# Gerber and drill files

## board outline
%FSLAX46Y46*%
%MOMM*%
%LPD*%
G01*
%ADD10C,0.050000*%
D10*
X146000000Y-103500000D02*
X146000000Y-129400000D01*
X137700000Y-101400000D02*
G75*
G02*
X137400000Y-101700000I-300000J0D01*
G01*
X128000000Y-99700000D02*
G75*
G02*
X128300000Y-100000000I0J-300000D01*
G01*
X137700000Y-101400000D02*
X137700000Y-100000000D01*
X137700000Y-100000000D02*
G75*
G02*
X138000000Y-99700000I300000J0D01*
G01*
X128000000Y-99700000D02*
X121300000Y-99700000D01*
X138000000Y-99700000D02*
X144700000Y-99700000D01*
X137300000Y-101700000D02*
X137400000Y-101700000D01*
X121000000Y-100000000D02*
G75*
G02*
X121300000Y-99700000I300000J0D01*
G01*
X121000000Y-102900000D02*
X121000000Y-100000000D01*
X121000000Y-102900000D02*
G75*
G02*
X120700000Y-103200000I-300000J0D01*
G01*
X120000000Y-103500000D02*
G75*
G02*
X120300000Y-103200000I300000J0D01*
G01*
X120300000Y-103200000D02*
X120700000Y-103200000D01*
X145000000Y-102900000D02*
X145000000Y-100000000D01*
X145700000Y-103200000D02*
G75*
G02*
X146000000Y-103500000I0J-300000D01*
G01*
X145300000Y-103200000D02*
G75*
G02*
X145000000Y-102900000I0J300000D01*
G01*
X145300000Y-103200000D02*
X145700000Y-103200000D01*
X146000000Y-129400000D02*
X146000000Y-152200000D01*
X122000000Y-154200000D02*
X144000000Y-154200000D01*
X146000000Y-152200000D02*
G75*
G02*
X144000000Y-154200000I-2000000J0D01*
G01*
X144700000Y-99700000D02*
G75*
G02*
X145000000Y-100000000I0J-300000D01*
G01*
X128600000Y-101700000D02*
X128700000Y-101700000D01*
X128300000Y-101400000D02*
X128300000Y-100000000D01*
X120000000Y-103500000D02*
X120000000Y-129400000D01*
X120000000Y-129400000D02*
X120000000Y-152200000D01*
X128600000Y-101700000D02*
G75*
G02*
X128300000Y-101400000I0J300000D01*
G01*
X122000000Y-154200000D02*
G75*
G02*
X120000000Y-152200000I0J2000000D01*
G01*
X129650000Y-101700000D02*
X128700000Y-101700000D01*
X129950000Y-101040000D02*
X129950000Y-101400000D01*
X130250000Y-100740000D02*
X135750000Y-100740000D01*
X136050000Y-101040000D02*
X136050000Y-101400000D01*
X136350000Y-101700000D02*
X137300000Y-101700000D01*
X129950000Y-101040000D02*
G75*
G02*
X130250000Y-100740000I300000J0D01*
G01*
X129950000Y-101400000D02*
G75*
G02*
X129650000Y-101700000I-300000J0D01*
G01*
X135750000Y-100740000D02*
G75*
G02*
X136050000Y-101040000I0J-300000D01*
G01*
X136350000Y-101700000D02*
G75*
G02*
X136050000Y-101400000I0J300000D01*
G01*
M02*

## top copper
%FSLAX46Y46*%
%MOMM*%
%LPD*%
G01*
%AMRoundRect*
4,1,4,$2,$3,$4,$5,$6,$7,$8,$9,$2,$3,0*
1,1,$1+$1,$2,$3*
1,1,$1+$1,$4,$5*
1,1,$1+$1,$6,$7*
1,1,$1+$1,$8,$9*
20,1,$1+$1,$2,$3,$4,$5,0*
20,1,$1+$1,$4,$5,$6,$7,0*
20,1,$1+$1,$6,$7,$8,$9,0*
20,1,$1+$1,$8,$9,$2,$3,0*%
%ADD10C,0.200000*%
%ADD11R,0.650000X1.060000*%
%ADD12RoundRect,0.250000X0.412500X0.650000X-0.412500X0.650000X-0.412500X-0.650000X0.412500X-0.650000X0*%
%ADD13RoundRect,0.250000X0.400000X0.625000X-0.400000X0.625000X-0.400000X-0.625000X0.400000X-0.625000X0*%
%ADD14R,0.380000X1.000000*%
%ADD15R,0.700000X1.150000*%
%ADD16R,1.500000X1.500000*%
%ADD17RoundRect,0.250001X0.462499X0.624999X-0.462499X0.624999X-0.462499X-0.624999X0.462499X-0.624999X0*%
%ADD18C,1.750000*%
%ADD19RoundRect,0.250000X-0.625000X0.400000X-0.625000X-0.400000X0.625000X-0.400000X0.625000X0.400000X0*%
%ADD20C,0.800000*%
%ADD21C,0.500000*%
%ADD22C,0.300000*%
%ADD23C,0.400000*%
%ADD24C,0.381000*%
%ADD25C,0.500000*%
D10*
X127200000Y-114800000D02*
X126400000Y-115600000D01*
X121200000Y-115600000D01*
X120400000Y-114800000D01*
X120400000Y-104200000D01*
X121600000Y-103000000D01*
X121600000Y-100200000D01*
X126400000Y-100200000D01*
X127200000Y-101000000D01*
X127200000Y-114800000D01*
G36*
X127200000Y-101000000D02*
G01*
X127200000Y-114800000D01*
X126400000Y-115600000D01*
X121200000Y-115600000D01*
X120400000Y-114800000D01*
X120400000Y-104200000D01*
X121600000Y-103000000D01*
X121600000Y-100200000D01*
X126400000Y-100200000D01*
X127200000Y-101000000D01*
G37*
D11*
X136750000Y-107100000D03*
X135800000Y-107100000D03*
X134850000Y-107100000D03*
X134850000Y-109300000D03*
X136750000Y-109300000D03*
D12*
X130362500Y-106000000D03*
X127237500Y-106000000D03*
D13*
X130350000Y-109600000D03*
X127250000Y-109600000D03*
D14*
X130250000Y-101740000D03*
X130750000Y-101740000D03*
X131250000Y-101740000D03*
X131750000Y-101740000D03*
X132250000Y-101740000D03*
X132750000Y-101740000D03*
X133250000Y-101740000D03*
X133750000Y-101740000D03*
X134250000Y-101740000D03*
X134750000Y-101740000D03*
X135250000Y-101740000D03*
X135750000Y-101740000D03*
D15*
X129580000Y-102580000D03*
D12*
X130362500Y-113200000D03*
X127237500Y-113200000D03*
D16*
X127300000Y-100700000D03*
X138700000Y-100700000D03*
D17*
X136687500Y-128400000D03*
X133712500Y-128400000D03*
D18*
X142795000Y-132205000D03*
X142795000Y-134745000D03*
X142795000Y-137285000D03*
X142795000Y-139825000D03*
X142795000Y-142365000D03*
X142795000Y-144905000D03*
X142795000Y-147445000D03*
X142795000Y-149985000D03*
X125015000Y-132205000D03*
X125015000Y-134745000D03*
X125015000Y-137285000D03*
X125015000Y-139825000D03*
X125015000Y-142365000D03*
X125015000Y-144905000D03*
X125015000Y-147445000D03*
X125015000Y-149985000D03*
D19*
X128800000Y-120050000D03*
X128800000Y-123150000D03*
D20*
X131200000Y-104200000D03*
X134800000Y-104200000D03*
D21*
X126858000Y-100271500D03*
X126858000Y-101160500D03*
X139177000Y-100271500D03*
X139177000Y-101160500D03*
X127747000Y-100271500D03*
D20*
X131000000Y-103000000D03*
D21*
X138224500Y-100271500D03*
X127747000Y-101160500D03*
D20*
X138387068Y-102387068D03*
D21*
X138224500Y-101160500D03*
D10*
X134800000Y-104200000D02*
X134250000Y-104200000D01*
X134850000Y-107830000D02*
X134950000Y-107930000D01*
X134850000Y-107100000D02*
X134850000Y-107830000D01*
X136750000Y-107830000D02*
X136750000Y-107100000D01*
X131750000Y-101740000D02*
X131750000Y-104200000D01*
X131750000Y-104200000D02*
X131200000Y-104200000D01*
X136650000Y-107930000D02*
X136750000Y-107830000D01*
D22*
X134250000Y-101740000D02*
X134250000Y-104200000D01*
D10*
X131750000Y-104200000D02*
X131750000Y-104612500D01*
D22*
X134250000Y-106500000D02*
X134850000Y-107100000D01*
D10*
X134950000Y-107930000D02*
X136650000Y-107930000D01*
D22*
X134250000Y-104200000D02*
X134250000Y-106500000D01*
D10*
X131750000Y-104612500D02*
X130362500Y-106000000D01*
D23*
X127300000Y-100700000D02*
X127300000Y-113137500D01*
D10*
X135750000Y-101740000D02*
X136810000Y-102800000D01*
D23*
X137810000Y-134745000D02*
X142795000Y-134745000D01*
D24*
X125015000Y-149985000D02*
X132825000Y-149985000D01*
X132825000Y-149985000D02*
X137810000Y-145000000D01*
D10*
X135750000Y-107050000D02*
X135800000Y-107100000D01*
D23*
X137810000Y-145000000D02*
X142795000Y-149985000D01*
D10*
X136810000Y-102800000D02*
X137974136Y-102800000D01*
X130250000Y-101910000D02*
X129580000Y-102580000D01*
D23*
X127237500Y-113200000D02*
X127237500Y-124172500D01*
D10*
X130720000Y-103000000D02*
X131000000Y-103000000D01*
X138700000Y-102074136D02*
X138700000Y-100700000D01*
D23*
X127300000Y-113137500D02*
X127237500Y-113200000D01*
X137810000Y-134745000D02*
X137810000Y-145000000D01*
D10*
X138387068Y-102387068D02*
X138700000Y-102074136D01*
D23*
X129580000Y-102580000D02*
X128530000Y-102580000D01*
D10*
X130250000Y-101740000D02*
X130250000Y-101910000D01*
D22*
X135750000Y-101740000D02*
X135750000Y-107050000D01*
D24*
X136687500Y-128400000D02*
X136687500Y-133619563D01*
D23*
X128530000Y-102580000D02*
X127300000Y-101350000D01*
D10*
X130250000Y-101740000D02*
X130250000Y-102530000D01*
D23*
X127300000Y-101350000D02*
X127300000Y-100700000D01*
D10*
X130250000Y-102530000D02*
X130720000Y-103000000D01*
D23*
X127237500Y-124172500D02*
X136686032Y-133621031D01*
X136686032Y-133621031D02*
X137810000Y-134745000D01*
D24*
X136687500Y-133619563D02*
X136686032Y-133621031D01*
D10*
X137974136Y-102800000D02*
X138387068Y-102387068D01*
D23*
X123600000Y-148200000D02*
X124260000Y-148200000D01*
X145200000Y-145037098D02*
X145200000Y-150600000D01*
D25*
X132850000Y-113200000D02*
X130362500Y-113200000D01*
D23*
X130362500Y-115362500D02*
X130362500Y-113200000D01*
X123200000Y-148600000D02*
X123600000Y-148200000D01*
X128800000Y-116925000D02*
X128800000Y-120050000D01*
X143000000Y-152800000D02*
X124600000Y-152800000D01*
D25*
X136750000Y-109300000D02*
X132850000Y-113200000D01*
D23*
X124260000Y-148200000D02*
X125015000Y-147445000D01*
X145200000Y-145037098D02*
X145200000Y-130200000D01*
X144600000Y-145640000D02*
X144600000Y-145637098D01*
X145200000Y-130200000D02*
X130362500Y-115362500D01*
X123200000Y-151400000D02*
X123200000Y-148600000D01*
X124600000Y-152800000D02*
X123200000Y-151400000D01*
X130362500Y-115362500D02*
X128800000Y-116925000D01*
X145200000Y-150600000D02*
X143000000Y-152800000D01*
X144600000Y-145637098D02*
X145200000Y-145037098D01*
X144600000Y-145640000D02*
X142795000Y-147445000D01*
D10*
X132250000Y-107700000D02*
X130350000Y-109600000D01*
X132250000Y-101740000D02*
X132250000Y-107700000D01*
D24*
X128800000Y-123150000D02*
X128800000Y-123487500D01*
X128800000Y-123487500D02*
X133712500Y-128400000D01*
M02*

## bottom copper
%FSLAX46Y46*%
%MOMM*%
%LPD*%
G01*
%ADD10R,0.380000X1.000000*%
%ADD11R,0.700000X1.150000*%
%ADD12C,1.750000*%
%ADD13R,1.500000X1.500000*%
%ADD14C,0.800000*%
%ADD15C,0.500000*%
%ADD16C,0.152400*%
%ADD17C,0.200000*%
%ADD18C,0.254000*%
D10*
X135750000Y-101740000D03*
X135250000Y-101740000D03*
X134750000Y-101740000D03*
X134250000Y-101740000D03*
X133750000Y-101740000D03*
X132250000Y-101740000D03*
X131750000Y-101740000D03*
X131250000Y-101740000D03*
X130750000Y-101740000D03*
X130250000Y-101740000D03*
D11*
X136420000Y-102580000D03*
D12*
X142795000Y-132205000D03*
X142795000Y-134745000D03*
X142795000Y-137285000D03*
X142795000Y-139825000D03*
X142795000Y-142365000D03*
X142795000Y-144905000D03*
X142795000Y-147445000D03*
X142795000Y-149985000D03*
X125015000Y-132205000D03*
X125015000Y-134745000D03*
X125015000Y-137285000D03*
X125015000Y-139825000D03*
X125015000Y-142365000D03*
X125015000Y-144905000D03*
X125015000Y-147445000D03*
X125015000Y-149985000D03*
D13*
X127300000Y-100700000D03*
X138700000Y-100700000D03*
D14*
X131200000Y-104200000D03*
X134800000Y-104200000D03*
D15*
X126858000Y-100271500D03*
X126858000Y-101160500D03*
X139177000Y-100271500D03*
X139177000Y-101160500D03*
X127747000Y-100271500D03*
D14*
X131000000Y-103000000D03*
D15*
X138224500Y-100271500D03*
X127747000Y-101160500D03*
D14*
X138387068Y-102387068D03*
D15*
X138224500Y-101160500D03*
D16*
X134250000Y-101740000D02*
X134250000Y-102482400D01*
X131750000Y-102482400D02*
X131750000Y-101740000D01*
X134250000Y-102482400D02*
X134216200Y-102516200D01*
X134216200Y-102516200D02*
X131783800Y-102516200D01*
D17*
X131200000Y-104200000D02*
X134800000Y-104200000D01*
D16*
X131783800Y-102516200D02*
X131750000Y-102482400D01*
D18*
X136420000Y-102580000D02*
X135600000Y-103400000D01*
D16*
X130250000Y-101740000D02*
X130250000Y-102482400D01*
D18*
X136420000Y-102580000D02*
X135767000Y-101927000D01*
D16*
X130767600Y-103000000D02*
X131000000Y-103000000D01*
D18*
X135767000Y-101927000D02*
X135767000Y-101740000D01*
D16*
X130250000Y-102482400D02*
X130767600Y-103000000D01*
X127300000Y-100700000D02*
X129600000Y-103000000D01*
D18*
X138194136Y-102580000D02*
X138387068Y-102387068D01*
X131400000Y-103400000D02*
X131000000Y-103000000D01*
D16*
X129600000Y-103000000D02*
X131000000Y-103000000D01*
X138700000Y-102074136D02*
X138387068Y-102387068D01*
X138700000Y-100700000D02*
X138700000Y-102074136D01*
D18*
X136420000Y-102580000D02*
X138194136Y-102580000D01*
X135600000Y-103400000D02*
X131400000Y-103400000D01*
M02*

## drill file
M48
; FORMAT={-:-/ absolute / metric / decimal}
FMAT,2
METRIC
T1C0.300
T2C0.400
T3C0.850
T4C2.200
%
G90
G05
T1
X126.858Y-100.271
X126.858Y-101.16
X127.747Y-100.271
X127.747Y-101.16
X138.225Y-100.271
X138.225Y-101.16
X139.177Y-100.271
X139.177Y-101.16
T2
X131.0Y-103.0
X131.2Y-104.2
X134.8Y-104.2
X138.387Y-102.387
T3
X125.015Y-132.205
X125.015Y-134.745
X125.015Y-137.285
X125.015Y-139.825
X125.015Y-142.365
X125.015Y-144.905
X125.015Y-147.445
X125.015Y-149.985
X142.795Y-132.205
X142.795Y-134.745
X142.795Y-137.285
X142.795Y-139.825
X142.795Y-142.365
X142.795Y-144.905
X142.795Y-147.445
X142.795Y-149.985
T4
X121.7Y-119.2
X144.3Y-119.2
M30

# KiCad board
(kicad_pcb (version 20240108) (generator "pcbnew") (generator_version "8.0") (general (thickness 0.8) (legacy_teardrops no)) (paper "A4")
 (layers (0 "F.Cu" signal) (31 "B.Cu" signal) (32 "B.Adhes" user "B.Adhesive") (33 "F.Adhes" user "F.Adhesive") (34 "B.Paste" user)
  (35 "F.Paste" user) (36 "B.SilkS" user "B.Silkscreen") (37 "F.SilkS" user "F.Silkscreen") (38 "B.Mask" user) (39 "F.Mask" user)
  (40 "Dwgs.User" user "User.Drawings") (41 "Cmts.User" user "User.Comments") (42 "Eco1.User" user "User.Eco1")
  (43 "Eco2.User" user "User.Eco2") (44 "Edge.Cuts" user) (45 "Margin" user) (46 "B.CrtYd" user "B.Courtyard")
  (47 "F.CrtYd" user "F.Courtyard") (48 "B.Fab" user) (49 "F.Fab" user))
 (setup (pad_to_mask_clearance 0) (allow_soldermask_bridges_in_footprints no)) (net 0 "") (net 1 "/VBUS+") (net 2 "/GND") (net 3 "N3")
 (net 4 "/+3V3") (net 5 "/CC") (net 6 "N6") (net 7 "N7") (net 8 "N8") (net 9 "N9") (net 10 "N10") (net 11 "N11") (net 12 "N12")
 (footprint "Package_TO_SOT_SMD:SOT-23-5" (layer "F.Cu") (at 135.8 108.2 -90)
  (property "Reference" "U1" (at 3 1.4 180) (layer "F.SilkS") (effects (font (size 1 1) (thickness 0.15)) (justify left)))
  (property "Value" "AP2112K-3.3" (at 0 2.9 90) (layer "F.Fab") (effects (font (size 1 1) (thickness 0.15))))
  (pad "1" smd rect (at -1.1 -0.95 270) (size 1.06 0.65) (layers "F.Cu" "F.Paste" "F.Mask") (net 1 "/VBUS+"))
  (pad "2" smd rect (at -1.1 0 270) (size 1.06 0.65) (layers "F.Cu" "F.Paste" "F.Mask") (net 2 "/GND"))
  (pad "3" smd rect (at -1.1 0.95 270) (size 1.06 0.65) (layers "F.Cu" "F.Paste" "F.Mask") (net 1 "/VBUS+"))
  (pad "4" smd rect (at 1.1 0.95 270) (size 1.06 0.65) (layers "F.Cu" "F.Paste" "F.Mask") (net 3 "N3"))
  (pad "5" smd rect (at 1.1 -0.95 270) (size 1.06 0.65) (layers "F.Cu" "F.Paste" "F.Mask") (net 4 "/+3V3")))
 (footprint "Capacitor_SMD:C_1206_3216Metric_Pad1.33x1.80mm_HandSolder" (layer "F.Cu") (at 128.8 106 180)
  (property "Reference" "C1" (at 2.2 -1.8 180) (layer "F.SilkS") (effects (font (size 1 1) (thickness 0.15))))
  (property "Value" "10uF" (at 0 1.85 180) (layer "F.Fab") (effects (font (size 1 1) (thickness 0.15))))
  (pad "1" smd roundrect (at -1.5625 0 180) (size 1.325 1.8) (layers "F.Cu" "F.Paste" "F.Mask") (roundrect_rratio 0.188679) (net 1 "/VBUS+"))
  (pad "2" smd roundrect (at 1.5625 0 180) (size 1.325 1.8) (layers "F.Cu" "F.Paste" "F.Mask") (roundrect_rratio 0.188679) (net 2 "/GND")))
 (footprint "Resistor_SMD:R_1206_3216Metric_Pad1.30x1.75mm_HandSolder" (layer "F.Cu") (at 128.8 109.6 180)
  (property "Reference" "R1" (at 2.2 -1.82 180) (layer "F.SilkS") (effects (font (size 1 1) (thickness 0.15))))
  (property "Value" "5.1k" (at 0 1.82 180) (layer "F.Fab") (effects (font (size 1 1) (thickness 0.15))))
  (pad "1" smd roundrect (at -1.55 0 180) (size 1.3 1.75) (layers "F.Cu" "F.Paste" "F.Mask") (roundrect_rratio 0.192308) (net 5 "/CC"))
  (pad "2" smd roundrect (at 1.55 0 180) (size 1.3 1.75) (layers "F.Cu" "F.Paste" "F.Mask") (roundrect_rratio 0.192308) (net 2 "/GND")))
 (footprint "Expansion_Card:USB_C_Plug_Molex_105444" (layer "F.Cu") (at 133 101.7)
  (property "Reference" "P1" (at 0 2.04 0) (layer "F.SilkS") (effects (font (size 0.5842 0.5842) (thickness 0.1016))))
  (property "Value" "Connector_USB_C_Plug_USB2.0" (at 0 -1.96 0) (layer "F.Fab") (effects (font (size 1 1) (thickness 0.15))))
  (fp_line (start -3.35 0) (end -4.3 0) (stroke (width 0.05) (type solid)) (layer "Edge.Cuts"))
  (fp_line (start -3.05 -0.66) (end -3.05 -0.3) (stroke (width 0.05) (type solid)) (layer "Edge.Cuts"))
  (fp_line (start -2.75 -0.96) (end 2.75 -0.96) (stroke (width 0.05) (type solid)) (layer "Edge.Cuts"))
  (fp_line (start 3.05 -0.66) (end 3.05 -0.3) (stroke (width 0.05) (type solid)) (layer "Edge.Cuts"))
  (fp_line (start 3.35 0) (end 4.3 0) (stroke (width 0.05) (type solid)) (layer "Edge.Cuts"))
  (fp_arc (start -3.05 -0.66) (mid -2.962132 -0.872132) (end -2.75 -0.96) (stroke (width 0.05) (type solid)) (layer "Edge.Cuts"))
  (fp_arc (start -3.05 -0.3) (mid -3.137868 -0.087868) (end -3.35 0) (stroke (width 0.05) (type solid)) (layer "Edge.Cuts"))
  (fp_arc (start 2.75 -0.96) (mid 2.962132 -0.872132) (end 3.05 -0.66) (stroke (width 0.05) (type solid)) (layer "Edge.Cuts"))
  (fp_arc (start 3.35 0) (mid 3.137868 -0.087868) (end 3.05 -0.3) (stroke (width 0.05) (type solid)) (layer "Edge.Cuts"))
  (pad "A1" smd rect (at -2.75 0.04) (size 0.38 1) (layers "F.Cu" "F.Paste" "F.Mask") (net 2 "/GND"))
  (pad "A2" smd rect (at -2.25 0.04) (size 0.38 1) (layers "F.Cu" "F.Paste" "F.Mask"))
  (pad "A3" smd rect (at -1.75 0.04) (size 0.38 1) (layers "F.Cu" "F.Paste" "F.Mask"))
  (pad "A4" smd rect (at -1.25 0.04) (size 0.38 1) (layers "F.Cu" "F.Paste" "F.Mask") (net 1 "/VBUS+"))
  (pad "A5" smd rect (at -0.75 0.04) (size 0.38 1) (layers "F.Cu" "F.Paste" "F.Mask") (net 5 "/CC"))
  (pad "A6" smd rect (at -0.25 0.04) (size 0.38 1) (layers "F.Cu" "F.Paste" "F.Mask") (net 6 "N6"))
  (pad "A7" smd rect (at 0.25 0.04) (size 0.38 1) (layers "F.Cu" "F.Paste" "F.Mask") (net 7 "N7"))
  (pad "A8" smd rect (at 0.75 0.04) (size 0.38 1) (layers "F.Cu" "F.Paste" "F.Mask"))
  (pad "A9" smd rect (at 1.25 0.04) (size 0.38 1) (layers "F.Cu" "F.Paste" "F.Mask") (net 1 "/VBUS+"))
  (pad "A10" smd rect (at 1.75 0.04) (size 0.38 1) (layers "F.Cu" "F.Paste" "F.Mask"))
  (pad "A11" smd rect (at 2.25 0.04) (size 0.38 1) (layers "F.Cu" "F.Paste" "F.Mask"))
  (pad "A12" smd rect (at 2.75 0.04) (size 0.38 1) (layers "F.Cu" "F.Paste" "F.Mask") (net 2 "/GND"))
  (pad "B1" smd rect (at 2.75 0.04) (size 0.38 1) (layers "B.Cu" "B.Paste" "B.Mask") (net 2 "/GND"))
  (pad "B2" smd rect (at 2.25 0.04) (size 0.38 1) (layers "B.Cu" "B.Paste" "B.Mask"))
  (pad "B3" smd rect (at 1.75 0.04) (size 0.38 1) (layers "B.Cu" "B.Paste" "B.Mask"))
  (pad "B4" smd rect (at 1.25 0.04) (size 0.38 1) (layers "B.Cu" "B.Paste" "B.Mask") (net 1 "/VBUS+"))
  (pad "B5" smd rect (at 0.75 0.04) (size 0.38 1) (layers "B.Cu" "B.Paste" "B.Mask") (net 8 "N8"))
  (pad "B8" smd rect (at -0.75 0.04) (size 0.38 1) (layers "B.Cu" "B.Paste" "B.Mask"))
  (pad "B9" smd rect (at -1.25 0.04) (size 0.38 1) (layers "B.Cu" "B.Paste" "B.Mask") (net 1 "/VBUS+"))
  (pad "B10" smd rect (at -1.75 0.04) (size 0.38 1) (layers "B.Cu" "B.Paste" "B.Mask"))
  (pad "B11" smd rect (at -2.25 0.04) (size 0.38 1) (layers "B.Cu" "B.Paste" "B.Mask"))
  (pad "B12" smd rect (at -2.75 0.04) (size 0.38 1) (layers "B.Cu" "B.Paste" "B.Mask") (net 2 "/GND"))
  (pad "S1" smd rect (at -3.42 0.88) (size 0.7 1.15) (layers "F.Cu" "F.Paste" "F.Mask") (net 2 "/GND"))
  (pad "S1" smd rect (at 3.42 0.88) (size 0.7 1.15) (layers "B.Cu" "B.Paste" "B.Mask") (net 2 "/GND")))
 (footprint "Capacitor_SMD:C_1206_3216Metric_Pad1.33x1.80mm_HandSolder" (layer "F.Cu") (at 128.8 113.2 180)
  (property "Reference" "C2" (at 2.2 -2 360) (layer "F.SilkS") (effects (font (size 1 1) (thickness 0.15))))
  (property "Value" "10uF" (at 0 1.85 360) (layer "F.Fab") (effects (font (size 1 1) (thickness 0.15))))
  (pad "1" smd roundrect (at -1.5625 0 180) (size 1.325 1.8) (layers "F.Cu" "F.Paste" "F.Mask") (roundrect_rratio 0.188679) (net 4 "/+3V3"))
  (pad "2" smd roundrect (at 1.5625 0 180) (size 1.325 1.8) (layers "F.Cu" "F.Paste" "F.Mask") (roundrect_rratio 0.188679) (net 2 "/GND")))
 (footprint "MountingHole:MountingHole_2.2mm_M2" (layer "F.Cu") (at 121.7 119.2)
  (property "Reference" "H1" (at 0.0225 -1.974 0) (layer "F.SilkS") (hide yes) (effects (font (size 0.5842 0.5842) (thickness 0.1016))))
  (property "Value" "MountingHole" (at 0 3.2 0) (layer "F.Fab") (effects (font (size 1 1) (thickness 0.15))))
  (pad "" np_thru_hole circle (at 0 0) (size 2.2 2.2) (drill 2.2) (layers "*.Cu" "*.Mask")))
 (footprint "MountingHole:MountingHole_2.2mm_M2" (layer "F.Cu") (at 144.3 119.2)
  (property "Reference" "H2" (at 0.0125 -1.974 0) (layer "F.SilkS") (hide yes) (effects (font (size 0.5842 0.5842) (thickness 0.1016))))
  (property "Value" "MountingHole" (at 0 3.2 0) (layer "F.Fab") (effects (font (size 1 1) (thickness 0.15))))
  (pad "" np_thru_hole circle (at 0 0) (size 2.2 2.2) (drill 2.2) (layers "*.Cu" "*.Mask")))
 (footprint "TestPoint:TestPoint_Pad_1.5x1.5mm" (layer "F.Cu") (at 127.3 100.7)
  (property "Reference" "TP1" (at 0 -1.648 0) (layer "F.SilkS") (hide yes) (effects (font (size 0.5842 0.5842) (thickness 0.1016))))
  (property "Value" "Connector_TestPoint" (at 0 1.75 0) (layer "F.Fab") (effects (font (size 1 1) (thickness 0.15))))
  (pad "1" smd rect (at 0 0) (size 1.5 1.5) (layers "F.Cu" "F.Mask") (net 2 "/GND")))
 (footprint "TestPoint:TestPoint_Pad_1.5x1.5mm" (layer "F.Cu") (at 138.7 100.7)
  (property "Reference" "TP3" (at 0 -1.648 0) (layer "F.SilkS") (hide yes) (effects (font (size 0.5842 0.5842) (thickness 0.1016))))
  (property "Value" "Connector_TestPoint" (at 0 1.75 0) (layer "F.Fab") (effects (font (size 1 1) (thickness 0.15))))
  (pad "1" smd rect (at 0 0) (size 1.5 1.5) (layers "F.Cu" "F.Mask") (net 2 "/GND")))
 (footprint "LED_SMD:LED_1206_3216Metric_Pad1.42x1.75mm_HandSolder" (layer "F.Cu") (at 135.2 128.4 180)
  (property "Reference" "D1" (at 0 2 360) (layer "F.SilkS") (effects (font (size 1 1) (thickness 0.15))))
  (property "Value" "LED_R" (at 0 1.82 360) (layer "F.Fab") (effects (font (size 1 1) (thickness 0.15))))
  (pad "1" smd roundrect (at -1.4875 0 180) (size 1.425 1.75) (layers "F.Cu" "F.Paste" "F.Mask") (roundrect_rratio 0.175439) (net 2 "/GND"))
  (pad "2" smd roundrect (at 1.4875 0 180) (size 1.425 1.75) (layers "F.Cu" "F.Paste" "F.Mask") (roundrect_rratio 0.175439) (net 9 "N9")))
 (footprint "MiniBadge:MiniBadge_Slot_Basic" (layer "F.Cu") (at 144.065 130.935 -90)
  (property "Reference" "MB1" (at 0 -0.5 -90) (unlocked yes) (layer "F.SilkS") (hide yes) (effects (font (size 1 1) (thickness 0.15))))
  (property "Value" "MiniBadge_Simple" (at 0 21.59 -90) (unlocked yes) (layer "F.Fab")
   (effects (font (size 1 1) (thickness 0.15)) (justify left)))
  (pad "1" thru_hole circle (at 1.27 1.27 270) (size 1.75 1.75) (drill 0.85) (layers "*.Cu" "*.Mask") (remove_unused_layers no)
   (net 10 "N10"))
  (pad "2" thru_hole circle (at 3.81 1.27 270) (size 1.75 1.75) (drill 0.85) (layers "*.Cu" "*.Mask") (remove_unused_layers no)
   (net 2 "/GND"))
  (pad "3" thru_hole circle (at 6.35 1.27 270) (size 1.75 1.75) (drill 0.85) (layers "*.Cu" "*.Mask") (remove_unused_layers no))
  (pad "4" thru_hole circle (at 8.89 1.27 270) (size 1.75 1.75) (drill 0.85) (layers "*.Cu" "*.Mask") (remove_unused_layers no))
  (pad "5" thru_hole circle (at 11.43 1.27 270) (size 1.75 1.75) (drill 0.85) (layers "*.Cu" "*.Mask") (remove_unused_layers no))
  (pad "6" thru_hole circle (at 13.97 1.27 270) (size 1.75 1.75) (drill 0.85) (layers "*.Cu" "*.Mask") (remove_unused_layers no))
  (pad "7" thru_hole circle (at 16.51 1.27 270) (size 1.75 1.75) (drill 0.85) (layers "*.Cu" "*.Mask") (remove_unused_layers no)
   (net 4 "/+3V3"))
  (pad "8" thru_hole circle (at 19.05 1.27 270) (size 1.75 1.75) (drill 0.85) (layers "*.Cu" "*.Mask") (remove_unused_layers no)
   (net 2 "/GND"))
  (pad "9" thru_hole circle (at 1.27 19.05 270) (size 1.75 1.75) (drill 0.85) (layers "*.Cu" "*.Mask") (remove_unused_layers no)
   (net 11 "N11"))
  (pad "10" thru_hole circle (at 3.81 19.05 270) (size 1.75 1.75) (drill 0.85) (layers "*.Cu" "*.Mask") (remove_unused_layers no)
   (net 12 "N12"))
  (pad "11" thru_hole circle (at 6.35 19.05 270) (size 1.75 1.75) (drill 0.85) (layers "*.Cu" "*.Mask") (remove_unused_layers no))
  (pad "12" thru_hole circle (at 8.89 19.05 270) (size 1.75 1.75) (drill 0.85) (layers "*.Cu" "*.Mask") (remove_unused_layers no))
  (pad "13" thru_hole circle (at 11.43 19.05 270) (size 1.75 1.75) (drill 0.85) (layers "*.Cu" "*.Mask") (remove_unused_layers no))
  (pad "14" thru_hole circle (at 13.97 19.05 270) (size 1.75 1.75) (drill 0.85) (layers "*.Cu" "*.Mask") (remove_unused_layers no))
  (pad "15" thru_hole circle (at 16.51 19.05 270) (size 1.75 1.75) (drill 0.85) (layers "*.Cu" "*.Mask") (remove_unused_layers no)
   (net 4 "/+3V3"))
  (pad "16" thru_hole circle (at 19.05 19.05 270) (size 1.75 1.75) (drill 0.85) (layers "*.Cu" "*.Mask") (remove_unused_layers no)
   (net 2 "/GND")))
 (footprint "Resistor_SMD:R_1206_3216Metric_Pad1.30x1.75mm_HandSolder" (layer "F.Cu") (at 128.8 121.6 -90)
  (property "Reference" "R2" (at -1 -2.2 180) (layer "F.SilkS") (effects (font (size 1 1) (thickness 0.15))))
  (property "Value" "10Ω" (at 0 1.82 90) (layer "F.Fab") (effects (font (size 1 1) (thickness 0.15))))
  (pad "1" smd roundrect (at -1.55 0 270) (size 1.3 1.75) (layers "F.Cu" "F.Paste" "F.Mask") (roundrect_rratio 0.192308) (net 4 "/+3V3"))
  (pad "2" smd roundrect (at 1.55 0 270) (size 1.3 1.75) (layers "F.Cu" "F.Paste" "F.Mask") (roundrect_rratio 0.192308) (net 9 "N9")))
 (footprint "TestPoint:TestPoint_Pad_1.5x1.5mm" (layer "B.Cu") (at 127.3 100.7)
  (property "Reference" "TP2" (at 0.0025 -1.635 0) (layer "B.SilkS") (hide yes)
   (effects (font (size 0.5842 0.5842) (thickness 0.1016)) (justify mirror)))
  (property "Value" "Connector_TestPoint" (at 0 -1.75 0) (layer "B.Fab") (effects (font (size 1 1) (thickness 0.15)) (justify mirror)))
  (pad "1" smd rect (at 0 0) (size 1.5 1.5) (layers "B.Cu" "B.Mask") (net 2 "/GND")))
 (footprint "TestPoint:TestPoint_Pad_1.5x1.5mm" (layer "B.Cu") (at 138.7 100.7)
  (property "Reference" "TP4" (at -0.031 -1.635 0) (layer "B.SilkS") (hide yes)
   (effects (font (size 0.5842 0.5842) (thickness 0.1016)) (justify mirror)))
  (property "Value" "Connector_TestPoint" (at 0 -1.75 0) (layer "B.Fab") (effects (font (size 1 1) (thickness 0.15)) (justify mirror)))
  (pad "1" smd rect (at 0 0) (size 1.5 1.5) (layers "B.Cu" "B.Mask") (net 2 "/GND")))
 (gr_poly
  (pts (xy 127.2 114.8) (xy 126.4 115.6) (xy 121.2 115.6) (xy 120.4 114.8) (xy 120.4 104.2) (xy 121.6 103) (xy 121.6 100.2) (xy 126.4 100.2)
   (xy 127.2 101))
  (stroke (width 0.2) (type solid)) (fill solid) (layer "F.Cu") (net 2))
 (gr_line (start 146 103.5) (end 146 129.4) (stroke (width 0.05) (type solid)) (layer "Edge.Cuts"))
 (gr_arc (start 137.7 101.4) (mid 137.612132 101.612132) (end 137.4 101.7) (stroke (width 0.05) (type solid)) (layer "Edge.Cuts"))
 (gr_arc (start 128 99.7) (mid 128.212132 99.787868) (end 128.3 100) (stroke (width 0.05) (type solid)) (layer "Edge.Cuts"))
 (gr_line (start 137.7 101.4) (end 137.7 100) (stroke (width 0.05) (type solid)) (layer "Edge.Cuts"))
 (gr_arc (start 137.7 100) (mid 137.787868 99.787868) (end 138 99.7) (stroke (width 0.05) (type solid)) (layer "Edge.Cuts"))
 (gr_line (start 128 99.7) (end 121.3 99.7) (stroke (width 0.05) (type solid)) (layer "Edge.Cuts"))
 (gr_line (start 138 99.7) (end 144.7 99.7) (stroke (width 0.05) (type solid)) (layer "Edge.Cuts"))
 (gr_line (start 137.3 101.7) (end 137.4 101.7) (stroke (width 0.05) (type solid)) (layer "Edge.Cuts"))
 (gr_arc (start 121 100) (mid 121.087868 99.787868) (end 121.3 99.7) (stroke (width 0.05) (type solid)) (layer "Edge.Cuts"))
 (gr_line (start 121 102.9) (end 121 100) (stroke (width 0.05) (type solid)) (layer "Edge.Cuts"))
 (gr_arc (start 121 102.9) (mid 120.912132 103.112132) (end 120.7 103.2) (stroke (width 0.05) (type solid)) (layer "Edge.Cuts"))
 (gr_arc (start 120 103.5) (mid 120.087868 103.287868) (end 120.3 103.2) (stroke (width 0.05) (type solid)) (layer "Edge.Cuts"))
 (gr_line (start 120.3 103.2) (end 120.7 103.2) (stroke (width 0.05) (type solid)) (layer "Edge.Cuts"))
 (gr_line (start 145 102.9) (end 145 100) (stroke (width 0.05) (type solid)) (layer "Edge.Cuts"))
 (gr_arc (start 145.7 103.2) (mid 145.912132 103.287868) (end 146 103.5) (stroke (width 0.05) (type solid)) (layer "Edge.Cuts"))
 (gr_arc (start 145.3 103.2) (mid 145.087868 103.112132) (end 145 102.9) (stroke (width 0.05) (type solid)) (layer "Edge.Cuts"))
 (gr_line (start 145.3 103.2) (end 145.7 103.2) (stroke (width 0.05) (type solid)) (layer "Edge.Cuts"))
 (gr_line (start 146 129.4) (end 146 152.2) (stroke (width 0.05) (type default)) (layer "Edge.Cuts"))
 (gr_line (start 122 154.2) (end 144 154.2) (stroke (width 0.05) (type default)) (layer "Edge.Cuts"))
 (gr_arc (start 146 152.2) (mid 145.414214 153.614214) (end 144 154.2) (stroke (width 0.05) (type default)) (layer "Edge.Cuts"))
 (gr_arc (start 144.7 99.7) (mid 144.912132 99.787868) (end 145 100) (stroke (width 0.05) (type solid)) (layer "Edge.Cuts"))
 (gr_line (start 128.6 101.7) (end 128.7 101.7) (stroke (width 0.05) (type solid)) (layer "Edge.Cuts"))
 (gr_line (start 128.3 101.4) (end 128.3 100) (stroke (width 0.05) (type solid)) (layer "Edge.Cuts"))
 (gr_line (start 120 103.5) (end 120 129.4) (stroke (width 0.05) (type solid)) (layer "Edge.Cuts"))
 (gr_line (start 120 129.4) (end 120 152.2) (stroke (width 0.05) (type default)) (layer "Edge.Cuts"))
 (gr_arc (start 128.6 101.7) (mid 128.387868 101.612132) (end 128.3 101.4) (stroke (width 0.05) (type solid)) (layer "Edge.Cuts"))
 (gr_arc (start 122 154.2) (mid 120.585786 153.614214) (end 120 152.2) (stroke (width 0.05) (type default)) (layer "Edge.Cuts"))
 (segment (start 134.8 104.2) (end 134.25 104.2) (width 0.2) (layer "F.Cu") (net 1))
 (segment (start 134.85 107.83) (end 134.95 107.93) (width 0.2) (layer "F.Cu") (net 1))
 (segment (start 134.85 107.1) (end 134.85 107.83) (width 0.2) (layer "F.Cu") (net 1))
 (segment (start 136.75 107.83) (end 136.75 107.1) (width 0.2) (layer "F.Cu") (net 1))
 (segment (start 131.75 101.74) (end 131.75 104.2) (width 0.2) (layer "F.Cu") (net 1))
 (segment (start 131.75 104.2) (end 131.2 104.2) (width 0.2) (layer "F.Cu") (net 1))
 (segment (start 136.65 107.93) (end 136.75 107.83) (width 0.2) (layer "F.Cu") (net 1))
 (segment (start 134.25 101.74) (end 134.25 104.2) (width 0.3) (layer "F.Cu") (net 1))
 (segment (start 131.75 104.2) (end 131.75 104.6125) (width 0.2) (layer "F.Cu") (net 1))
 (segment (start 134.25 106.5) (end 134.85 107.1) (width 0.3) (layer "F.Cu") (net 1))
 (segment (start 134.95 107.93) (end 136.65 107.93) (width 0.2) (layer "F.Cu") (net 1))
 (segment (start 134.25 104.2) (end 134.25 106.5) (width 0.3) (layer "F.Cu") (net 1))
 (segment (start 131.75 104.6125) (end 130.3625 106) (width 0.2) (layer "F.Cu") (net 1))
 (via (at 131.2 104.2) (size 0.8) (drill 0.4) (layers "F.Cu" "B.Cu") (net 1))
 (via (at 134.8 104.2) (size 0.8) (drill 0.4) (layers "F.Cu" "B.Cu") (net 1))
 (segment (start 134.25 101.74) (end 134.25 102.4824) (width 0.1524) (layer "B.Cu") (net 1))
 (segment (start 131.75 102.4824) (end 131.75 101.74) (width 0.1524) (layer "B.Cu") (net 1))
 (segment (start 134.25 102.4824) (end 134.2162 102.5162) (width 0.1524) (layer "B.Cu") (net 1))
 (segment (start 134.2162 102.5162) (end 131.7838 102.5162) (width 0.1524) (layer "B.Cu") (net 1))
 (segment (start 131.2 104.2) (end 134.8 104.2) (width 0.2) (layer "B.Cu") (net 1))
 (segment (start 131.7838 102.5162) (end 131.75 102.4824) (width 0.1524) (layer "B.Cu") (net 1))
 (segment (start 127.3 100.7) (end 127.3 113.1375) (width 0.4) (layer "F.Cu") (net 2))
 (segment (start 135.75 101.74) (end 136.81 102.8) (width 0.2) (layer "F.Cu") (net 2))
 (segment (start 137.81 134.745) (end 142.795 134.745) (width 0.4) (layer "F.Cu") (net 2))
 (segment (start 125.015 149.985) (end 132.825 149.985) (width 0.381) (layer "F.Cu") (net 2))
 (segment (start 132.825 149.985) (end 137.81 145) (width 0.381) (layer "F.Cu") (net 2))
 (segment (start 135.75 107.05) (end 135.8 107.1) (width 0.2) (layer "F.Cu") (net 2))
 (segment (start 137.81 145) (end 142.795 149.985) (width 0.4) (layer "F.Cu") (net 2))
 (segment (start 136.81 102.8) (end 137.974136 102.8) (width 0.2) (layer "F.Cu") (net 2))
 (segment (start 130.25 101.91) (end 129.58 102.58) (width 0.2) (layer "F.Cu") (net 2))
 (segment (start 127.2375 113.2) (end 127.2375 124.1725) (width 0.4) (layer "F.Cu") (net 2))
 (segment (start 130.72 103) (end 131 103) (width 0.2) (layer "F.Cu") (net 2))
 (segment (start 138.7 102.074136) (end 138.7 100.7) (width 0.2) (layer "F.Cu") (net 2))
 (segment (start 127.3 113.1375) (end 127.2375 113.2) (width 0.4) (layer "F.Cu") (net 2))
 (segment (start 137.81 134.745) (end 137.81 145) (width 0.4) (layer "F.Cu") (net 2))
 (segment (start 138.387068 102.387068) (end 138.7 102.074136) (width 0.2) (layer "F.Cu") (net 2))
 (segment (start 129.58 102.58) (end 128.53 102.58) (width 0.4) (layer "F.Cu") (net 2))
 (segment (start 130.25 101.74) (end 130.25 101.91) (width 0.2) (layer "F.Cu") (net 2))
 (segment (start 135.75 101.74) (end 135.75 107.05) (width 0.3) (layer "F.Cu") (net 2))
 (segment (start 136.6875 128.4) (end 136.6875 133.619563) (width 0.381) (layer "F.Cu") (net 2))
 (segment (start 128.53 102.58) (end 127.3 101.35) (width 0.4) (layer "F.Cu") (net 2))
 (segment (start 130.25 101.74) (end 130.25 102.53) (width 0.2) (layer "F.Cu") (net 2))
 (segment (start 127.3 101.35) (end 127.3 100.7) (width 0.4) (layer "F.Cu") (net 2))
 (segment (start 130.25 102.53) (end 130.72 103) (width 0.2) (layer "F.Cu") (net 2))
 (segment (start 127.2375 124.1725) (end 136.686032 133.621031) (width 0.4) (layer "F.Cu") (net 2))
 (segment (start 136.686032 133.621031) (end 137.81 134.745) (width 0.4) (layer "F.Cu") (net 2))
 (segment (start 136.6875 133.619563) (end 136.686032 133.621031) (width 0.381) (layer "F.Cu") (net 2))
 (segment (start 137.974136 102.8) (end 138.387068 102.387068) (width 0.2) (layer "F.Cu") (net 2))
 (via (at 126.858 100.2715) (size 0.5) (drill 0.3) (layers "F.Cu" "B.Cu") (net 2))
 (via (at 126.858 101.1605) (size 0.5) (drill 0.3) (layers "F.Cu" "B.Cu") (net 2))
 (via (at 139.177 100.2715) (size 0.5) (drill 0.3) (layers "F.Cu" "B.Cu") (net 2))
 (via (at 139.177 101.1605) (size 0.5) (drill 0.3) (layers "F.Cu" "B.Cu") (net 2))
 (via (at 127.747 100.2715) (size 0.5) (drill 0.3) (layers "F.Cu" "B.Cu") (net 2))
 (via (at 131 103) (size 0.8) (drill 0.4) (layers "F.Cu" "B.Cu") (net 2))
 (via (at 138.2245 100.2715) (size 0.5) (drill 0.3) (layers "F.Cu" "B.Cu") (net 2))
 (via (at 127.747 101.1605) (size 0.5) (drill 0.3) (layers "F.Cu" "B.Cu") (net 2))
 (via (at 138.387068 102.387068) (size 0.8) (drill 0.4) (layers "F.Cu" "B.Cu") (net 2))
 (via (at 138.2245 101.1605) (size 0.5) (drill 0.3) (layers "F.Cu" "B.Cu") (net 2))
 (segment (start 136.42 102.58) (end 135.6 103.4) (width 0.254) (layer "B.Cu") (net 2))
 (segment (start 130.25 101.74) (end 130.25 102.4824) (width 0.1524) (layer "B.Cu") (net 2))
 (segment (start 136.42 102.58) (end 135.767 101.927) (width 0.254) (layer "B.Cu") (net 2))
 (segment (start 130.7676 103) (end 131 103) (width 0.1524) (layer "B.Cu") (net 2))
 (segment (start 135.767 101.927) (end 135.767 101.74) (width 0.254) (layer "B.Cu") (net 2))
 (segment (start 130.25 102.4824) (end 130.7676 103) (width 0.1524) (layer "B.Cu") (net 2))
 (segment (start 127.3 100.7) (end 129.6 103) (width 0.1524) (layer "B.Cu") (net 2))
 (segment (start 138.194136 102.58) (end 138.387068 102.387068) (width 0.254) (layer "B.Cu") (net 2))
 (segment (start 131.4 103.4) (end 131 103) (width 0.254) (layer "B.Cu") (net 2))
 (segment (start 129.6 103) (end 131 103) (width 0.1524) (layer "B.Cu") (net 2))
 (segment (start 138.7 102.074136) (end 138.387068 102.387068) (width 0.1524) (layer "B.Cu") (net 2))
 (segment (start 138.7 100.7) (end 138.7 102.074136) (width 0.1524) (layer "B.Cu") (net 2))
 (segment (start 136.42 102.58) (end 138.194136 102.58) (width 0.254) (layer "B.Cu") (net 2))
 (segment (start 135.6 103.4) (end 131.4 103.4) (width 0.254) (layer "B.Cu") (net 2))
 (segment (start 123.6 148.2) (end 124.26 148.2) (width 0.4) (layer "F.Cu") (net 4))
 (segment (start 145.2 145.037098) (end 145.2 150.6) (width 0.4) (layer "F.Cu") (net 4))
 (segment (start 132.85 113.2) (end 130.3625 113.2) (width 0.5) (layer "F.Cu") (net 4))
 (segment (start 130.3625 115.3625) (end 130.3625 113.2) (width 0.4) (layer "F.Cu") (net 4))
 (segment (start 123.2 148.6) (end 123.6 148.2) (width 0.4) (layer "F.Cu") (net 4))
 (segment (start 128.8 116.925) (end 128.8 120.05) (width 0.4) (layer "F.Cu") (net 4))
 (segment (start 143 152.8) (end 124.6 152.8) (width 0.4) (layer "F.Cu") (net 4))
 (segment (start 136.75 109.3) (end 132.85 113.2) (width 0.5) (layer "F.Cu") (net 4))
 (segment (start 124.26 148.2) (end 125.015 147.445) (width 0.4) (layer "F.Cu") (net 4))
 (segment (start 145.2 145.037098) (end 145.2 130.2) (width 0.4) (layer "F.Cu") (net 4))
 (segment (start 144.6 145.64) (end 144.6 145.637098) (width 0.4) (layer "F.Cu") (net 4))
 (segment (start 145.2 130.2) (end 130.3625 115.3625) (width 0.4) (layer "F.Cu") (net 4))
 (segment (start 123.2 151.4) (end 123.2 148.6) (width 0.4) (layer "F.Cu") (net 4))
 (segment (start 124.6 152.8) (end 123.2 151.4) (width 0.4) (layer "F.Cu") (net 4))
 (segment (start 130.3625 115.3625) (end 128.8 116.925) (width 0.4) (layer "F.Cu") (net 4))
 (segment (start 145.2 150.6) (end 143 152.8) (width 0.4) (layer "F.Cu") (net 4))
 (segment (start 144.6 145.637098) (end 145.2 145.037098) (width 0.4) (layer "F.Cu") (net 4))
 (segment (start 144.6 145.64) (end 142.795 147.445) (width 0.4) (layer "F.Cu") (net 4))
 (segment (start 132.25 107.7) (end 130.35 109.6) (width 0.2) (layer "F.Cu") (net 5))
 (segment (start 132.25 101.74) (end 132.25 107.7) (width 0.2) (layer "F.Cu") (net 5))
 (segment (start 128.8 123.15) (end 128.8 123.4875) (width 0.381) (layer "F.Cu") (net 9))
 (segment (start 128.8 123.4875) (end 133.7125 128.4) (width 0.381) (layer "F.Cu") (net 9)))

